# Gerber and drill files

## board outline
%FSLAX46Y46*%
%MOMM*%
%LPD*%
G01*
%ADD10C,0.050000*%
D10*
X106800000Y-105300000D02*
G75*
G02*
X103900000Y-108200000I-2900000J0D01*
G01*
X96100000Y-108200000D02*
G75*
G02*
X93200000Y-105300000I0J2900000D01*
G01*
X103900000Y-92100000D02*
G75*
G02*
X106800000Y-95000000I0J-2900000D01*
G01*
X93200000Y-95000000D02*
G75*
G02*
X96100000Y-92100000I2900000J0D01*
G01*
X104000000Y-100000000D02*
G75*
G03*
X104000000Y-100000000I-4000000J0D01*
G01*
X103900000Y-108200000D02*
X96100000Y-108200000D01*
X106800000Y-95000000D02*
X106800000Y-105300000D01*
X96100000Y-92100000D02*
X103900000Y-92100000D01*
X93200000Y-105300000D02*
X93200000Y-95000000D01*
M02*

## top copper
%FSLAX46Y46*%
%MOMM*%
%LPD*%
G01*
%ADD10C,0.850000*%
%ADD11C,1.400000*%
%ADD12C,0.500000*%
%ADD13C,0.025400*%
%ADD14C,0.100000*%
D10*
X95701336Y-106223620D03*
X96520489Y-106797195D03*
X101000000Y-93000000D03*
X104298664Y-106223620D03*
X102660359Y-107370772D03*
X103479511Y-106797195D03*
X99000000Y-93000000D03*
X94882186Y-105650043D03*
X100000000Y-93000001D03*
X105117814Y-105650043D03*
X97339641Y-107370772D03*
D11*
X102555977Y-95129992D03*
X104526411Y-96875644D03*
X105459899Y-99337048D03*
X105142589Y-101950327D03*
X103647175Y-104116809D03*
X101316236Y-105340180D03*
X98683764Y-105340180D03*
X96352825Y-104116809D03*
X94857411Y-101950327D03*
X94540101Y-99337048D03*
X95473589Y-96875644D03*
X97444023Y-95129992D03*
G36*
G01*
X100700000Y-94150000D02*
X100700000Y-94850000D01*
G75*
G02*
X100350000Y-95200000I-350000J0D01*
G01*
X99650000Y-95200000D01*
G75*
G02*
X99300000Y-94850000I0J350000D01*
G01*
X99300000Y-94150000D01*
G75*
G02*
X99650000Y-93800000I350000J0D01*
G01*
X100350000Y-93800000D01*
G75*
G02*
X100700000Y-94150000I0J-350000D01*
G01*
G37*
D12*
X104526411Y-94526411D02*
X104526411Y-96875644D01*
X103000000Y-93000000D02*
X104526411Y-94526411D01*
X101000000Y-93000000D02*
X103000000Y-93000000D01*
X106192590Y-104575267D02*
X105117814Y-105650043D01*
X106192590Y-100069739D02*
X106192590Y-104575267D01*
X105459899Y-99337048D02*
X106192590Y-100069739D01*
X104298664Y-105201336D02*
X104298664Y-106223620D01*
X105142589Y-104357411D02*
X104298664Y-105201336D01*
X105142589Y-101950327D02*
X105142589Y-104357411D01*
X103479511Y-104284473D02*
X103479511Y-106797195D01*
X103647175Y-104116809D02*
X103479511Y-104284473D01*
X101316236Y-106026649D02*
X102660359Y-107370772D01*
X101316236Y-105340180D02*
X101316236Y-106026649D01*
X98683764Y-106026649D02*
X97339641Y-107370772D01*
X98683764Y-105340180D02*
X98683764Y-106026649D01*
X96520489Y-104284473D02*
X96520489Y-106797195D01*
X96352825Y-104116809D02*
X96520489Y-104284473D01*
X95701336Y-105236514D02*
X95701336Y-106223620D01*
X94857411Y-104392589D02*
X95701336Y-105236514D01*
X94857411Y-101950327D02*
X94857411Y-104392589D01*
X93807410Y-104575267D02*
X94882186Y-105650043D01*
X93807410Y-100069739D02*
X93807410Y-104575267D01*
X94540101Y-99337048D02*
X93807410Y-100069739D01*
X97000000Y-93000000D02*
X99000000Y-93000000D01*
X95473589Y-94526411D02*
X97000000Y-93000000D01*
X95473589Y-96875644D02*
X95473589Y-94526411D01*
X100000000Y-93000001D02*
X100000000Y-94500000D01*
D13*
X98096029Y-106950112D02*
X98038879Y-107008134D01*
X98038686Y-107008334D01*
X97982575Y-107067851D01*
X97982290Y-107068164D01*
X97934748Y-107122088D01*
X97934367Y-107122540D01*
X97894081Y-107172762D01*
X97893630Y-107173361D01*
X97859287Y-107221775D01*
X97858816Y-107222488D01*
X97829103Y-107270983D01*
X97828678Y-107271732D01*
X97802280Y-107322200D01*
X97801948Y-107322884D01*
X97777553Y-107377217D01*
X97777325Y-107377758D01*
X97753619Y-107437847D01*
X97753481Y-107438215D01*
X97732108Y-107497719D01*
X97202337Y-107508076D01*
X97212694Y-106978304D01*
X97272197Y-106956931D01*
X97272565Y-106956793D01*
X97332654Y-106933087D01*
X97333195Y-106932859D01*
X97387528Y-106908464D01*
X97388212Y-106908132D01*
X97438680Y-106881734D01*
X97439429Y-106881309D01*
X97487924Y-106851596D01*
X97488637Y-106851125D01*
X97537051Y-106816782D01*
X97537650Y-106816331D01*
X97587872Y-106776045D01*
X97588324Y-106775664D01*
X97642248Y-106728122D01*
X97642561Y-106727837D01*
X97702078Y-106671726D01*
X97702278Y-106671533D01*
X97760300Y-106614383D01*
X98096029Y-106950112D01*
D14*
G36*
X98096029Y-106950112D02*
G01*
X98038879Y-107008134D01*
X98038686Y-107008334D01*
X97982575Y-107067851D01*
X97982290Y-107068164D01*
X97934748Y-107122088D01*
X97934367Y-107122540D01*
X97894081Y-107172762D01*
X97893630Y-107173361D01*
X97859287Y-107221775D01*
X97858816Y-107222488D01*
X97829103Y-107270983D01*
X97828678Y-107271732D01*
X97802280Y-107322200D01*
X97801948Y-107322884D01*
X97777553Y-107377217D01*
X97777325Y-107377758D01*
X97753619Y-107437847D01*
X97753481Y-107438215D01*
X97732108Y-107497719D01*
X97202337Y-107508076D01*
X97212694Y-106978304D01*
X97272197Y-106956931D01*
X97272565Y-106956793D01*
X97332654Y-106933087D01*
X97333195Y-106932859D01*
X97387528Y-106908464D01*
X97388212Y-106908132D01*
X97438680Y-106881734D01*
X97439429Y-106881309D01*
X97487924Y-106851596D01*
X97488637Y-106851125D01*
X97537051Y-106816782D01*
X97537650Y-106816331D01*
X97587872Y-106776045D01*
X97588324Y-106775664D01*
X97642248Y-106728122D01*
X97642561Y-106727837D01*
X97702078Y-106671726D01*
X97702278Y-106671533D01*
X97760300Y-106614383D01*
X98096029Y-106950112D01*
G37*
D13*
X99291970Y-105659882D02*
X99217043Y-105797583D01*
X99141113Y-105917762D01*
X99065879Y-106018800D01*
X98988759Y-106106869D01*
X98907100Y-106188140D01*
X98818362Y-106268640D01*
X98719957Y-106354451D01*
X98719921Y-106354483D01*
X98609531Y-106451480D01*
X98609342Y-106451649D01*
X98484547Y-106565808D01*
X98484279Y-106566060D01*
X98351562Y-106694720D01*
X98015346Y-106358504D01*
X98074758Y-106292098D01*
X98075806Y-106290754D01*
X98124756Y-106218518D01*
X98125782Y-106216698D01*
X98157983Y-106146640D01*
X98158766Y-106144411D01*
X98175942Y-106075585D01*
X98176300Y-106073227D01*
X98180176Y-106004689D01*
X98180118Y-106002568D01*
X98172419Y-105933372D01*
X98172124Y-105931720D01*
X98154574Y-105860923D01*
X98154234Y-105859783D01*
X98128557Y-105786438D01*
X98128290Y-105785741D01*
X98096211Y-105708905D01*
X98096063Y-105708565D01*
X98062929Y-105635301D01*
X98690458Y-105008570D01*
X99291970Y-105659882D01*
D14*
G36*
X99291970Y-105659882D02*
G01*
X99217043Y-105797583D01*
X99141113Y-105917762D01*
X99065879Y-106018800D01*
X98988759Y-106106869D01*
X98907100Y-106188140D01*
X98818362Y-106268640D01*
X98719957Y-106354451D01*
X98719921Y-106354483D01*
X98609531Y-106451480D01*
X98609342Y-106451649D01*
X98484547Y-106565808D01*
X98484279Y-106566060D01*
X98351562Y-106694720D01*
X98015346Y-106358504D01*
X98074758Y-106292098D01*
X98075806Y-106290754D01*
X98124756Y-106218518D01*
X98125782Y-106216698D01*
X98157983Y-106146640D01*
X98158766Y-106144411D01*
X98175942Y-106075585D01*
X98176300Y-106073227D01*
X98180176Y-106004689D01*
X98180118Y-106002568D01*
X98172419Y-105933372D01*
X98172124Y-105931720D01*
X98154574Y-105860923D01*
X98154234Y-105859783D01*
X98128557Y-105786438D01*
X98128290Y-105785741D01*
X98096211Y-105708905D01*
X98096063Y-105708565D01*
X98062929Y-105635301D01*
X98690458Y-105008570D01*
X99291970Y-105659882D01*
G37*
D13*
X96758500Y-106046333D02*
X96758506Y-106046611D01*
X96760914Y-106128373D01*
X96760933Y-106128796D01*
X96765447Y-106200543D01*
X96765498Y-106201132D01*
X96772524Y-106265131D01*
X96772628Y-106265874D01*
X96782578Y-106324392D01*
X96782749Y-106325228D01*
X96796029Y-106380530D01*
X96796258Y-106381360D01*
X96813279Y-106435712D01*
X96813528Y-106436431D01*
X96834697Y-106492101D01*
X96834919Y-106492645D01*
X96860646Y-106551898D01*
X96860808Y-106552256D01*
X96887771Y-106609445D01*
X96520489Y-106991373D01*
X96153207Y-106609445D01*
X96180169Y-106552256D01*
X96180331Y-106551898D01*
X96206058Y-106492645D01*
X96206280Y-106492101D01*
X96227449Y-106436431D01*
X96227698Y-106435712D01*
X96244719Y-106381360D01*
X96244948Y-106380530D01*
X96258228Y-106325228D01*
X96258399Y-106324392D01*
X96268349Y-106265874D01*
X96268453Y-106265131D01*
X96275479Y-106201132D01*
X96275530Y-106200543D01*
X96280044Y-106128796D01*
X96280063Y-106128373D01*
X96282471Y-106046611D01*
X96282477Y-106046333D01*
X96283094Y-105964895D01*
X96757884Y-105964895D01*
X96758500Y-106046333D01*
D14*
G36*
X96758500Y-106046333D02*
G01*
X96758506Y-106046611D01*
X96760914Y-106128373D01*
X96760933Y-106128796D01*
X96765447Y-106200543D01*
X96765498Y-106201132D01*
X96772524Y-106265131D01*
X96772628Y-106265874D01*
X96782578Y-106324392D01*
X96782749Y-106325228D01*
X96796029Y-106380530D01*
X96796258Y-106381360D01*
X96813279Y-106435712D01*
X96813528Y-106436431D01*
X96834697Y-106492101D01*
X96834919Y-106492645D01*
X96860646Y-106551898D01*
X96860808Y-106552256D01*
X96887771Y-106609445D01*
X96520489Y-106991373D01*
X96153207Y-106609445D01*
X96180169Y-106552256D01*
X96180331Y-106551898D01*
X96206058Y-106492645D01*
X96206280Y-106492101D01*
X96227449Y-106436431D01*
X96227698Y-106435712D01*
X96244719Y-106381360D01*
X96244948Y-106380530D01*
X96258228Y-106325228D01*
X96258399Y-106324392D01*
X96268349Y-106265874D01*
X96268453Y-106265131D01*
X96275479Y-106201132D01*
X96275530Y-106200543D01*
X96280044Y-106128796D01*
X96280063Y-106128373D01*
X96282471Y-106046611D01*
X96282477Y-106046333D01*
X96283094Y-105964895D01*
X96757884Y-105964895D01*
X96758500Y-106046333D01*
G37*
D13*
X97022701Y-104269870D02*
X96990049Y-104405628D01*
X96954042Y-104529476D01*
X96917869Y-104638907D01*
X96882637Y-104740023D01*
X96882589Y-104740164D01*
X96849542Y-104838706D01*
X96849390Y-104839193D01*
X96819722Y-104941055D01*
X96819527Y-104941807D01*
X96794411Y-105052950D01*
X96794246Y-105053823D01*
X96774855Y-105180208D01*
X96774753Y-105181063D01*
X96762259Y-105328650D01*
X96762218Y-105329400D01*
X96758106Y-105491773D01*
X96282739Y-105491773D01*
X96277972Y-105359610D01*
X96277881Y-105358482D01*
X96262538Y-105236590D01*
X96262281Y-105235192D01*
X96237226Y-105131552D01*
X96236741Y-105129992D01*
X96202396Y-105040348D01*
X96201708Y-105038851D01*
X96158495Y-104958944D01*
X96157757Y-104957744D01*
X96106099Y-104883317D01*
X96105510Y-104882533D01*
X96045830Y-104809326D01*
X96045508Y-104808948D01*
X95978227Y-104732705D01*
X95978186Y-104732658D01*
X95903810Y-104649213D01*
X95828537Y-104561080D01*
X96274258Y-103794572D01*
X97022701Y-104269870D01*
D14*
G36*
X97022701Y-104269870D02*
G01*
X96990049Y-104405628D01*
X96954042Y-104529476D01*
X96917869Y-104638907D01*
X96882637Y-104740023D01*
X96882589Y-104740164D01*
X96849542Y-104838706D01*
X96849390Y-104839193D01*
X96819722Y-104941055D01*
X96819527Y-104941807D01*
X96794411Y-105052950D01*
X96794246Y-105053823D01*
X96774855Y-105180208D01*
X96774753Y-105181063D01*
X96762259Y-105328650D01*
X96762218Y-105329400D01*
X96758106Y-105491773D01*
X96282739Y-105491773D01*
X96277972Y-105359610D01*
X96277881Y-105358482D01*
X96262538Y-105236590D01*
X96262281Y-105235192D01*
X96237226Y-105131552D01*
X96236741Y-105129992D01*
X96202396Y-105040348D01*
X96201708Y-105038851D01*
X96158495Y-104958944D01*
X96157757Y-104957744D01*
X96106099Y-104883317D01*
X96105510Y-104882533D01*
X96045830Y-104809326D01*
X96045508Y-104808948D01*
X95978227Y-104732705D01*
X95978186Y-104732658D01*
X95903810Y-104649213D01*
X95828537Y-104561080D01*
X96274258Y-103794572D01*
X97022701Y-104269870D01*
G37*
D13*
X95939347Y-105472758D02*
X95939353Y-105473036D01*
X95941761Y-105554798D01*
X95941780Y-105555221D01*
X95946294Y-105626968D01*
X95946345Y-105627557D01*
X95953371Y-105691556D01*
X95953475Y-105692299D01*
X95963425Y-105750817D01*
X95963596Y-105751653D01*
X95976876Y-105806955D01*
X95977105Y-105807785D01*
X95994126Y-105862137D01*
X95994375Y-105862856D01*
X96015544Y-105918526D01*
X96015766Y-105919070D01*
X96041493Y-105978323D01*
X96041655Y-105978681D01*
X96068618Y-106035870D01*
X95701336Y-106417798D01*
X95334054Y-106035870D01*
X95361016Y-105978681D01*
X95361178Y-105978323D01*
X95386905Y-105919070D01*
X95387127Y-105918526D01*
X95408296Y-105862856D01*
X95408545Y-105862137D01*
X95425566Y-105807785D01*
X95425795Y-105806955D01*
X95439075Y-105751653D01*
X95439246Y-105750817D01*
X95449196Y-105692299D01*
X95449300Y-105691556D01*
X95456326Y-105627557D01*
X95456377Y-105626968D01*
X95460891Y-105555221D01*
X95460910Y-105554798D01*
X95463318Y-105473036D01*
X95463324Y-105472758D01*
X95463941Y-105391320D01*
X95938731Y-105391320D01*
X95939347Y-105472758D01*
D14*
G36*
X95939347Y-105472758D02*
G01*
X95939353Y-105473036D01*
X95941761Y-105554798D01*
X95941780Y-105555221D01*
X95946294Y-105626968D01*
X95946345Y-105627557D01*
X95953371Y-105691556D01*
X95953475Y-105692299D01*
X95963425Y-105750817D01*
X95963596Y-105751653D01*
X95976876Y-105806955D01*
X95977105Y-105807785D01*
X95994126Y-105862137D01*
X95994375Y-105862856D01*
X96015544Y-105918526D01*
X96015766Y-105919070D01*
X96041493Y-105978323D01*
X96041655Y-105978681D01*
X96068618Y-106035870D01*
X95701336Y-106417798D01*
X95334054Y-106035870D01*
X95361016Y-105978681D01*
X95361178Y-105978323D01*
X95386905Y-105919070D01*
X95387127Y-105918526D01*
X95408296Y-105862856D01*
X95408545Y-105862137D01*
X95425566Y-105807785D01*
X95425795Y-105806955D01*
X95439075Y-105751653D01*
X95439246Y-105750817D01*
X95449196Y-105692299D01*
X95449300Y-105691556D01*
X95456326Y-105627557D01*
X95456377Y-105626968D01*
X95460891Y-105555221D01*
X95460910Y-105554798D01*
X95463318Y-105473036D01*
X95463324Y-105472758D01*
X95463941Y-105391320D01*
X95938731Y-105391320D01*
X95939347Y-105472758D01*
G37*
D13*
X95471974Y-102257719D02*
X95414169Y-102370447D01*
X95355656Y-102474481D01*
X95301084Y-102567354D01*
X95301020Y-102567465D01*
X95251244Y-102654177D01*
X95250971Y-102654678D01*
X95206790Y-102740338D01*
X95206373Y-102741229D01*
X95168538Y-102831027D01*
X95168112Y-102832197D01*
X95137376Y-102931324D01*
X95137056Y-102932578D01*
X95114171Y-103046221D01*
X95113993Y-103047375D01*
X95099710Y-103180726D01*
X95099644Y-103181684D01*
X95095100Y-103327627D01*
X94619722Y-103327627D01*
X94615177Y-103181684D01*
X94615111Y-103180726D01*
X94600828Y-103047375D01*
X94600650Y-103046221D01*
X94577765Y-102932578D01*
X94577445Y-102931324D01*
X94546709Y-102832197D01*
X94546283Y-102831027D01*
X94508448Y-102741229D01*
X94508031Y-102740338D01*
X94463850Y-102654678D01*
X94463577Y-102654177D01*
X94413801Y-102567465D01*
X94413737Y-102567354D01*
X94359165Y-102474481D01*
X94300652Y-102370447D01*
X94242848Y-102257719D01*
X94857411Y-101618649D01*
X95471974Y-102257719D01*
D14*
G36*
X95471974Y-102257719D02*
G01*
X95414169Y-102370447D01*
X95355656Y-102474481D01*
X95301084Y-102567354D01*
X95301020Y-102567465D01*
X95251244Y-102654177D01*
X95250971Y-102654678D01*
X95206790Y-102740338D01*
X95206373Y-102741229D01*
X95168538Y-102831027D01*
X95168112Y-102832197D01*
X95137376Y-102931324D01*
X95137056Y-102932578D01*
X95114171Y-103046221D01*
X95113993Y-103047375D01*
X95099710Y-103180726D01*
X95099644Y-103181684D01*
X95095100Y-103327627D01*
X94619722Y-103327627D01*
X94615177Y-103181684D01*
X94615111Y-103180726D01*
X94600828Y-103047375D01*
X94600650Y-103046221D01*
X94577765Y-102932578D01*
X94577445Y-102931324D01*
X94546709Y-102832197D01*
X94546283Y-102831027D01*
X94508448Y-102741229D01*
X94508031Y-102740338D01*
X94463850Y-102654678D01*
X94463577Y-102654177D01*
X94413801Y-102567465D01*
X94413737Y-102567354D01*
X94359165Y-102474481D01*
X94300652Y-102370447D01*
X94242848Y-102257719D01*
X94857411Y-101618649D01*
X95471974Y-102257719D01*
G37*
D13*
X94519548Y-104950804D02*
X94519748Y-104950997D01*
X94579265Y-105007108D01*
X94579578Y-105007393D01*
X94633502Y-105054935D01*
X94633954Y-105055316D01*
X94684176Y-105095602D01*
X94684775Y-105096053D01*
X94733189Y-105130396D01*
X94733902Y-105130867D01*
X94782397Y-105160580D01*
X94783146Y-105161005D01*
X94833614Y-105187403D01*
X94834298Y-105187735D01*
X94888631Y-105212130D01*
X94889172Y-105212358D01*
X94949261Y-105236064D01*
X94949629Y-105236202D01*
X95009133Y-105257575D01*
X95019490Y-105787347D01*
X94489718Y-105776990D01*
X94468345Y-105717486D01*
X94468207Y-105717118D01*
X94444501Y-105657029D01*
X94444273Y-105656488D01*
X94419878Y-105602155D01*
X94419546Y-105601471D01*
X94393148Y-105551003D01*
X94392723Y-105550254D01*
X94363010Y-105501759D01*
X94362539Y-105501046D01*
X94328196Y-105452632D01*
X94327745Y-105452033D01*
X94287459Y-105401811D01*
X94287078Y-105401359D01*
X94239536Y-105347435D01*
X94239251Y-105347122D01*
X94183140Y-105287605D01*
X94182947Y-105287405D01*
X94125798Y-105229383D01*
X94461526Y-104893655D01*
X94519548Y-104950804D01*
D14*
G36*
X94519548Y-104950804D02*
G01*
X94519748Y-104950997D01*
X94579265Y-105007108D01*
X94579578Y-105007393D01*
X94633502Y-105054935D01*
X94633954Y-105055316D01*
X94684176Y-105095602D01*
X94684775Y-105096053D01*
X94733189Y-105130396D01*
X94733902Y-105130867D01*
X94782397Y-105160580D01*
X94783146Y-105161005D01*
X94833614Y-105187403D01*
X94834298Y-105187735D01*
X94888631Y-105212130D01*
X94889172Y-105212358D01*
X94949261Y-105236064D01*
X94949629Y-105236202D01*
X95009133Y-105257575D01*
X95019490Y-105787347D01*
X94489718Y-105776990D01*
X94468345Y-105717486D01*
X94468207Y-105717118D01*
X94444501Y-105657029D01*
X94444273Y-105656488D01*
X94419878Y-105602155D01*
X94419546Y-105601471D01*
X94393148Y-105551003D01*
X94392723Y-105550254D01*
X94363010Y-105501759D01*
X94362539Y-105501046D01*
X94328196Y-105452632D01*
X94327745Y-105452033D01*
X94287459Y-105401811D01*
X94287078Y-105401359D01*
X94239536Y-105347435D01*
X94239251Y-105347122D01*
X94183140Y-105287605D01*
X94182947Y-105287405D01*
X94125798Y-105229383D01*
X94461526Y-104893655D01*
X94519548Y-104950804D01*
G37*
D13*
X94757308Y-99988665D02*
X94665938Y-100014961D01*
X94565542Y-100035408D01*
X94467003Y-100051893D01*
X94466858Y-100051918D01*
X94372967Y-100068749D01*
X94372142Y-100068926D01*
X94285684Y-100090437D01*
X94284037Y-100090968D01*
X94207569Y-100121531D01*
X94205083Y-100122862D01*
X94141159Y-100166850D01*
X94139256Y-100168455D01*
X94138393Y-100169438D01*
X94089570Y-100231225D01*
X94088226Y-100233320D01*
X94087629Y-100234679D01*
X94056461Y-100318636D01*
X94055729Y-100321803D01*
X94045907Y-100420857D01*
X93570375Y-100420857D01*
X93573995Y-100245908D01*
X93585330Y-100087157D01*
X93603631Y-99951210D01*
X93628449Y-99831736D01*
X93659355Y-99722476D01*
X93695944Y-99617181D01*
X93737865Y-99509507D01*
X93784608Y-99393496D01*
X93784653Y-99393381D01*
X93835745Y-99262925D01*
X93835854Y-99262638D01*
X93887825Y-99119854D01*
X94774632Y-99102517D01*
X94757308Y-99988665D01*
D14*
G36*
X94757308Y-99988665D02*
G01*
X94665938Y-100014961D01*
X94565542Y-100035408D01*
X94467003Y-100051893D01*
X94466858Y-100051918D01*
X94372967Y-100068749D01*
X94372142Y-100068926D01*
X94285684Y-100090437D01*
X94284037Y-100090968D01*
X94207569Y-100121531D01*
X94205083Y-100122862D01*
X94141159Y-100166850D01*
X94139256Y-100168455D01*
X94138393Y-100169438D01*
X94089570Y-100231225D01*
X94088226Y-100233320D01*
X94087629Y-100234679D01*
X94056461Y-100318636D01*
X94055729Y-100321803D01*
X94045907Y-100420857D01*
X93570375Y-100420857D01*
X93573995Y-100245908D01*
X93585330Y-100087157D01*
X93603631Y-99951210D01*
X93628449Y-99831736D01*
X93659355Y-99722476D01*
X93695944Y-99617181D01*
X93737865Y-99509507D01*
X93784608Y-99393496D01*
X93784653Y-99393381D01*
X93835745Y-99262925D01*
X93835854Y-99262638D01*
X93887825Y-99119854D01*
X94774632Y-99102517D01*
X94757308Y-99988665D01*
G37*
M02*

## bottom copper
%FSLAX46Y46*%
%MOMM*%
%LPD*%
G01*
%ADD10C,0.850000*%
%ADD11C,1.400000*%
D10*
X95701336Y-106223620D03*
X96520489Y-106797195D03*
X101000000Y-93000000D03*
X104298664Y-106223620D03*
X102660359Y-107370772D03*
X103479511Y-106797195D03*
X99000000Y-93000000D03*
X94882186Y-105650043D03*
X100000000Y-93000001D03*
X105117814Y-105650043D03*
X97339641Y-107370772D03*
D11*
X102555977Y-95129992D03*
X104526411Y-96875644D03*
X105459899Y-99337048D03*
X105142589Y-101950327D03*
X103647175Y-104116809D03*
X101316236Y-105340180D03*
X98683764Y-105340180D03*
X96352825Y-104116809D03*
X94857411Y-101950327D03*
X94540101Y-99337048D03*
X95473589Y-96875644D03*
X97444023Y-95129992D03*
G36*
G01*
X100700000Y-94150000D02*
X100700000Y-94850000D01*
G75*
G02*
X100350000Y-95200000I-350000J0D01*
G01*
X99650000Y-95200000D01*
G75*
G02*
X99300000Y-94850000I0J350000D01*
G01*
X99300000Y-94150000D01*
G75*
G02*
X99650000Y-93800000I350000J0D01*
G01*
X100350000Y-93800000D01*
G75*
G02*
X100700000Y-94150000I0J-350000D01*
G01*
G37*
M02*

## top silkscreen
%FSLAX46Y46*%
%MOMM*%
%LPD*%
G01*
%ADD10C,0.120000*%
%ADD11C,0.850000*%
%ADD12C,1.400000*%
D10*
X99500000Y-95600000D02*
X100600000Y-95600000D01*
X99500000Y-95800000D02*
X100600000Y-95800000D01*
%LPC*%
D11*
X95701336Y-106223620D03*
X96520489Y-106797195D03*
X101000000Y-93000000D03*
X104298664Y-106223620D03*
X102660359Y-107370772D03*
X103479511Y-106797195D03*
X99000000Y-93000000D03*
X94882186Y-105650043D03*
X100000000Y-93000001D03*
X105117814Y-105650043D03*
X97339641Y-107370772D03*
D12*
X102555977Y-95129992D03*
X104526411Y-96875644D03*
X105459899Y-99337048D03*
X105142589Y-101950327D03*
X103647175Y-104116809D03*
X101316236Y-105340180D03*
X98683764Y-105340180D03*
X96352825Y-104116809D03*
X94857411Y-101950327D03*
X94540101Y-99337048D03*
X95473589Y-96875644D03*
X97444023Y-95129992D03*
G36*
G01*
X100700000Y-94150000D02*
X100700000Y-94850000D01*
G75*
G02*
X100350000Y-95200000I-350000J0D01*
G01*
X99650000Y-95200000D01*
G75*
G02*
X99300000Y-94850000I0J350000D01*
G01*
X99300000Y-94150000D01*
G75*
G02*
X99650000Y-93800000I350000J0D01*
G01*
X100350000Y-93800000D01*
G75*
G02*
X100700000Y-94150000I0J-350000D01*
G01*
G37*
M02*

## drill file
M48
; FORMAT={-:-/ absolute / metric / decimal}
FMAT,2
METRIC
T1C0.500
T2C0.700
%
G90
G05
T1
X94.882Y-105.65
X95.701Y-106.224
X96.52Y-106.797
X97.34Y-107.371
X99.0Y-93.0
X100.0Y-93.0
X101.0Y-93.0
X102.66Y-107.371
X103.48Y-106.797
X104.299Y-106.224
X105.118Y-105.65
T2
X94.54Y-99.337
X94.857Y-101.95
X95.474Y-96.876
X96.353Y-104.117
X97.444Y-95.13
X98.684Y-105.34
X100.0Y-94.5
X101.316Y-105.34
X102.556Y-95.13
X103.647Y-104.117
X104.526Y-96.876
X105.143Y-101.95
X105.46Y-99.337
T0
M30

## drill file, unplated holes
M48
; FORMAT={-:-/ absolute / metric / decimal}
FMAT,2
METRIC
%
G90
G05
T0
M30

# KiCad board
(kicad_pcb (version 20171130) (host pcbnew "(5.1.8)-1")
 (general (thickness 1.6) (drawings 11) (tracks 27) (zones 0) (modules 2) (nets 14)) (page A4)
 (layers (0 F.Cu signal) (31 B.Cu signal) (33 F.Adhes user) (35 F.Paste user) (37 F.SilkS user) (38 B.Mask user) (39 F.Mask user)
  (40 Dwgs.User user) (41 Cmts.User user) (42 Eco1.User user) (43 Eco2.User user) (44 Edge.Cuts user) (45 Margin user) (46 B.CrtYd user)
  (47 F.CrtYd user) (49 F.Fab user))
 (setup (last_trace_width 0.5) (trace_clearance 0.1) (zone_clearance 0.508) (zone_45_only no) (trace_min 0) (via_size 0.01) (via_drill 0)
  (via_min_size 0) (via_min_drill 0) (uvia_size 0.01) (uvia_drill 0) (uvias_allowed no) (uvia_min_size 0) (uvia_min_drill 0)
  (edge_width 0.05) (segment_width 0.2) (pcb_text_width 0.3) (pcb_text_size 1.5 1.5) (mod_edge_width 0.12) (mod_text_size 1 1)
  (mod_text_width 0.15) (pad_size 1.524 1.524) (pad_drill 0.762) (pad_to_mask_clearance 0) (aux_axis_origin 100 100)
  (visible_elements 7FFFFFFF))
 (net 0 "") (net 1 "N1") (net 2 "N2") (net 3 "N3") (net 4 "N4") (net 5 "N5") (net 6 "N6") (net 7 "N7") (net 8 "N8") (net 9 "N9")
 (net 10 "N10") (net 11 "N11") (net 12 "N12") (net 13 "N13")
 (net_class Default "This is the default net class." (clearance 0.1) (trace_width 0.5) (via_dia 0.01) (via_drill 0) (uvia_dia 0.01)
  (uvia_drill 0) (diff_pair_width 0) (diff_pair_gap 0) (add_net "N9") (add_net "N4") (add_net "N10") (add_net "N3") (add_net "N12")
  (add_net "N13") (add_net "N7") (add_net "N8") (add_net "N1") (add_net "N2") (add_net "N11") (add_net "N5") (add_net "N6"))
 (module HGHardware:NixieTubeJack (layer F.Cu) (at 100 100)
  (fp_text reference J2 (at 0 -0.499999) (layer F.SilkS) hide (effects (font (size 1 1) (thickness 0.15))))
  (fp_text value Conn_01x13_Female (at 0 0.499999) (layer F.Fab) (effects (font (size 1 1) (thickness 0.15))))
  (pad 5 thru_hole circle (at -4.298664 6.22362 325) (size 0.85 0.85) (drill 0.5) (layers *.Cu *.Mask) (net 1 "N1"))
  (pad 6 thru_hole circle (at -3.479511 6.797195 235) (size 0.85 0.85) (drill 0.5) (layers *.Cu *.Mask) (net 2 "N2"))
  (pad 12 thru_hole circle (at 1 -7 270) (size 0.85 0.85) (drill 0.5) (layers *.Cu *.Mask) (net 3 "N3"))
  (pad 10 thru_hole circle (at 4.298664 6.22362 230) (size 0.85 0.85) (drill 0.5) (layers *.Cu *.Mask) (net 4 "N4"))
  (pad 8 thru_hole circle (at 2.660359 7.370772 140) (size 0.85 0.85) (drill 0.5) (layers *.Cu *.Mask) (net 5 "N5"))
  (pad 9 thru_hole circle (at 3.479511 6.797195 140) (size 0.85 0.85) (drill 0.5) (layers *.Cu *.Mask) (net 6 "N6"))
  (pad 3 thru_hole circle (at -1 -7 270) (size 0.85 0.85) (drill 0.5) (layers *.Cu *.Mask) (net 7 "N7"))
  (pad 4 thru_hole circle (at -5.117814 5.650043 325) (size 0.85 0.85) (drill 0.5) (layers *.Cu *.Mask) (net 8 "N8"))
  (pad 1 thru_hole circle (at 0 -6.999999 180) (size 0.85 0.85) (drill 0.5) (layers *.Cu *.Mask) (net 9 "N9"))
  (pad 11 thru_hole circle (at 5.117814 5.650043 230) (size 0.85 0.85) (drill 0.5) (layers *.Cu *.Mask) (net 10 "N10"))
  (pad 7 thru_hole circle (at -2.660359 7.370772 235) (size 0.85 0.85) (drill 0.5) (layers *.Cu *.Mask) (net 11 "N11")))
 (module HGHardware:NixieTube (layer F.Cu) (at 100 100 180)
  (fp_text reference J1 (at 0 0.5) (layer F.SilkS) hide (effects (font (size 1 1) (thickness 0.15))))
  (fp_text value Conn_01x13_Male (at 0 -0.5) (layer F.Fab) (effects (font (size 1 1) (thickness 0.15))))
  (pad 13 thru_hole circle (at -2.555977 4.870008 180) (size 1.4 1.4) (drill 0.7) (layers *.Cu *.Mask) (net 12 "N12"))
  (pad 12 thru_hole circle (at -4.526411 3.124356 180) (size 1.4 1.4) (drill 0.7) (layers *.Cu *.Mask) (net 3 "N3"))
  (pad 11 thru_hole circle (at -5.459899 0.662952 180) (size 1.4 1.4) (drill 0.7) (layers *.Cu *.Mask) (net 10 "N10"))
  (pad 10 thru_hole circle (at -5.142589 -1.950327 180) (size 1.4 1.4) (drill 0.7) (layers *.Cu *.Mask) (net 4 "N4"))
  (pad 9 thru_hole circle (at -3.647175 -4.116809 180) (size 1.4 1.4) (drill 0.7) (layers *.Cu *.Mask) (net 6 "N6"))
  (pad 8 thru_hole circle (at -1.316236 -5.34018 180) (size 1.4 1.4) (drill 0.7) (layers *.Cu *.Mask) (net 5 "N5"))
  (pad 7 thru_hole circle (at 1.316236 -5.34018 180) (size 1.4 1.4) (drill 0.7) (layers *.Cu *.Mask) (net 11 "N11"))
  (pad 6 thru_hole circle (at 3.647175 -4.116809 180) (size 1.4 1.4) (drill 0.7) (layers *.Cu *.Mask) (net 2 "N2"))
  (pad 5 thru_hole circle (at 5.142589 -1.950327 180) (size 1.4 1.4) (drill 0.7) (layers *.Cu *.Mask) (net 1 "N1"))
  (pad 4 thru_hole circle (at 5.459899 0.662952 180) (size 1.4 1.4) (drill 0.7) (layers *.Cu *.Mask) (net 8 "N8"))
  (pad 3 thru_hole circle (at 4.526411 3.124356 180) (size 1.4 1.4) (drill 0.7) (layers *.Cu *.Mask) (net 7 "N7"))
  (pad 2 thru_hole circle (at 2.555977 4.870008 180) (size 1.4 1.4) (drill 0.7) (layers *.Cu *.Mask) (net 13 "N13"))
  (pad 1 thru_hole roundrect (at 0 5.5 180) (size 1.4 1.4) (drill 0.7) (layers *.Cu *.Mask) (roundrect_rratio 0.25) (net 9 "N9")))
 (gr_arc (start 103.9 105.3) (end 103.9 108.2) (angle -90) (layer Edge.Cuts) (width 0.05))
 (gr_arc (start 96.1 105.3) (end 93.2 105.3) (angle -90) (layer Edge.Cuts) (width 0.05))
 (gr_arc (start 103.9 95) (end 106.8 95) (angle -90) (layer Edge.Cuts) (width 0.05))
 (gr_arc (start 96.1 95) (end 96.1 92.1) (angle -90) (layer Edge.Cuts) (width 0.05))
 (gr_circle (center 100 100) (end 104 100) (layer Edge.Cuts) (width 0.05))
 (gr_line (start 103.9 108.2) (end 96.1 108.2) (layer Edge.Cuts) (width 0.05))
 (gr_line (start 106.8 95) (end 106.8 105.3) (layer Edge.Cuts) (width 0.05))
 (gr_line (start 96.1 92.1) (end 103.9 92.1) (layer Edge.Cuts) (width 0.05))
 (gr_line (start 93.2 105.3) (end 93.2 95) (layer Edge.Cuts) (width 0.05))
 (gr_line (start 99.5 95.6) (end 100.6 95.6) (layer F.SilkS) (width 0.12))
 (gr_line (start 99.5 95.8) (end 100.6 95.8) (layer F.SilkS) (width 0.12))
 (segment (start 104.526411 94.526411) (end 104.526411 96.875644) (width 0.5) (layer F.Cu) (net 3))
 (segment (start 103 93) (end 104.526411 94.526411) (width 0.5) (layer F.Cu) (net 3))
 (segment (start 101 93) (end 103 93) (width 0.5) (layer F.Cu) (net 3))
 (segment (start 106.19259 104.575267) (end 105.117814 105.650043) (width 0.5) (layer F.Cu) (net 10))
 (segment (start 106.19259 100.069739) (end 106.19259 104.575267) (width 0.5) (layer F.Cu) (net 10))
 (segment (start 105.459899 99.337048) (end 106.19259 100.069739) (width 0.5) (layer F.Cu) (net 10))
 (segment (start 104.298664 105.201336) (end 104.298664 106.22362) (width 0.5) (layer F.Cu) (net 4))
 (segment (start 105.142589 104.357411) (end 104.298664 105.201336) (width 0.5) (layer F.Cu) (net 4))
 (segment (start 105.142589 101.950327) (end 105.142589 104.357411) (width 0.5) (layer F.Cu) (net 4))
 (segment (start 103.479511 104.284473) (end 103.479511 106.797195) (width 0.5) (layer F.Cu) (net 6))
 (segment (start 103.647175 104.116809) (end 103.479511 104.284473) (width 0.5) (layer F.Cu) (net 6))
 (segment (start 101.316236 106.026649) (end 102.660359 107.370772) (width 0.5) (layer F.Cu) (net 5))
 (segment (start 101.316236 105.34018) (end 101.316236 106.026649) (width 0.5) (layer F.Cu) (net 5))
 (segment (start 98.683764 106.026649) (end 97.339641 107.370772) (width 0.5) (layer F.Cu) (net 11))
 (segment (start 98.683764 105.34018) (end 98.683764 106.026649) (width 0.5) (layer F.Cu) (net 11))
 (segment (start 96.520489 104.284473) (end 96.520489 106.797195) (width 0.5) (layer F.Cu) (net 2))
 (segment (start 96.352825 104.116809) (end 96.520489 104.284473) (width 0.5) (layer F.Cu) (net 2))
 (segment (start 95.701336 105.236514) (end 95.701336 106.22362) (width 0.5) (layer F.Cu) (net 1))
 (segment (start 94.857411 104.392589) (end 95.701336 105.236514) (width 0.5) (layer F.Cu) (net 1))
 (segment (start 94.857411 101.950327) (end 94.857411 104.392589) (width 0.5) (layer F.Cu) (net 1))
 (segment (start 93.80741 104.575267) (end 94.882186 105.650043) (width 0.5) (layer F.Cu) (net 8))
 (segment (start 93.80741 100.069739) (end 93.80741 104.575267) (width 0.5) (layer F.Cu) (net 8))
 (segment (start 94.540101 99.337048) (end 93.80741 100.069739) (width 0.5) (layer F.Cu) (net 8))
 (segment (start 97 93) (end 99 93) (width 0.5) (layer F.Cu) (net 7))
 (segment (start 95.473589 94.526411) (end 97 93) (width 0.5) (layer F.Cu) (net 7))
 (segment (start 95.473589 96.875644) (end 95.473589 94.526411) (width 0.5) (layer F.Cu) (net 7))
 (segment (start 100 93.000001) (end 100 94.5) (width 0.5) (layer F.Cu) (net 9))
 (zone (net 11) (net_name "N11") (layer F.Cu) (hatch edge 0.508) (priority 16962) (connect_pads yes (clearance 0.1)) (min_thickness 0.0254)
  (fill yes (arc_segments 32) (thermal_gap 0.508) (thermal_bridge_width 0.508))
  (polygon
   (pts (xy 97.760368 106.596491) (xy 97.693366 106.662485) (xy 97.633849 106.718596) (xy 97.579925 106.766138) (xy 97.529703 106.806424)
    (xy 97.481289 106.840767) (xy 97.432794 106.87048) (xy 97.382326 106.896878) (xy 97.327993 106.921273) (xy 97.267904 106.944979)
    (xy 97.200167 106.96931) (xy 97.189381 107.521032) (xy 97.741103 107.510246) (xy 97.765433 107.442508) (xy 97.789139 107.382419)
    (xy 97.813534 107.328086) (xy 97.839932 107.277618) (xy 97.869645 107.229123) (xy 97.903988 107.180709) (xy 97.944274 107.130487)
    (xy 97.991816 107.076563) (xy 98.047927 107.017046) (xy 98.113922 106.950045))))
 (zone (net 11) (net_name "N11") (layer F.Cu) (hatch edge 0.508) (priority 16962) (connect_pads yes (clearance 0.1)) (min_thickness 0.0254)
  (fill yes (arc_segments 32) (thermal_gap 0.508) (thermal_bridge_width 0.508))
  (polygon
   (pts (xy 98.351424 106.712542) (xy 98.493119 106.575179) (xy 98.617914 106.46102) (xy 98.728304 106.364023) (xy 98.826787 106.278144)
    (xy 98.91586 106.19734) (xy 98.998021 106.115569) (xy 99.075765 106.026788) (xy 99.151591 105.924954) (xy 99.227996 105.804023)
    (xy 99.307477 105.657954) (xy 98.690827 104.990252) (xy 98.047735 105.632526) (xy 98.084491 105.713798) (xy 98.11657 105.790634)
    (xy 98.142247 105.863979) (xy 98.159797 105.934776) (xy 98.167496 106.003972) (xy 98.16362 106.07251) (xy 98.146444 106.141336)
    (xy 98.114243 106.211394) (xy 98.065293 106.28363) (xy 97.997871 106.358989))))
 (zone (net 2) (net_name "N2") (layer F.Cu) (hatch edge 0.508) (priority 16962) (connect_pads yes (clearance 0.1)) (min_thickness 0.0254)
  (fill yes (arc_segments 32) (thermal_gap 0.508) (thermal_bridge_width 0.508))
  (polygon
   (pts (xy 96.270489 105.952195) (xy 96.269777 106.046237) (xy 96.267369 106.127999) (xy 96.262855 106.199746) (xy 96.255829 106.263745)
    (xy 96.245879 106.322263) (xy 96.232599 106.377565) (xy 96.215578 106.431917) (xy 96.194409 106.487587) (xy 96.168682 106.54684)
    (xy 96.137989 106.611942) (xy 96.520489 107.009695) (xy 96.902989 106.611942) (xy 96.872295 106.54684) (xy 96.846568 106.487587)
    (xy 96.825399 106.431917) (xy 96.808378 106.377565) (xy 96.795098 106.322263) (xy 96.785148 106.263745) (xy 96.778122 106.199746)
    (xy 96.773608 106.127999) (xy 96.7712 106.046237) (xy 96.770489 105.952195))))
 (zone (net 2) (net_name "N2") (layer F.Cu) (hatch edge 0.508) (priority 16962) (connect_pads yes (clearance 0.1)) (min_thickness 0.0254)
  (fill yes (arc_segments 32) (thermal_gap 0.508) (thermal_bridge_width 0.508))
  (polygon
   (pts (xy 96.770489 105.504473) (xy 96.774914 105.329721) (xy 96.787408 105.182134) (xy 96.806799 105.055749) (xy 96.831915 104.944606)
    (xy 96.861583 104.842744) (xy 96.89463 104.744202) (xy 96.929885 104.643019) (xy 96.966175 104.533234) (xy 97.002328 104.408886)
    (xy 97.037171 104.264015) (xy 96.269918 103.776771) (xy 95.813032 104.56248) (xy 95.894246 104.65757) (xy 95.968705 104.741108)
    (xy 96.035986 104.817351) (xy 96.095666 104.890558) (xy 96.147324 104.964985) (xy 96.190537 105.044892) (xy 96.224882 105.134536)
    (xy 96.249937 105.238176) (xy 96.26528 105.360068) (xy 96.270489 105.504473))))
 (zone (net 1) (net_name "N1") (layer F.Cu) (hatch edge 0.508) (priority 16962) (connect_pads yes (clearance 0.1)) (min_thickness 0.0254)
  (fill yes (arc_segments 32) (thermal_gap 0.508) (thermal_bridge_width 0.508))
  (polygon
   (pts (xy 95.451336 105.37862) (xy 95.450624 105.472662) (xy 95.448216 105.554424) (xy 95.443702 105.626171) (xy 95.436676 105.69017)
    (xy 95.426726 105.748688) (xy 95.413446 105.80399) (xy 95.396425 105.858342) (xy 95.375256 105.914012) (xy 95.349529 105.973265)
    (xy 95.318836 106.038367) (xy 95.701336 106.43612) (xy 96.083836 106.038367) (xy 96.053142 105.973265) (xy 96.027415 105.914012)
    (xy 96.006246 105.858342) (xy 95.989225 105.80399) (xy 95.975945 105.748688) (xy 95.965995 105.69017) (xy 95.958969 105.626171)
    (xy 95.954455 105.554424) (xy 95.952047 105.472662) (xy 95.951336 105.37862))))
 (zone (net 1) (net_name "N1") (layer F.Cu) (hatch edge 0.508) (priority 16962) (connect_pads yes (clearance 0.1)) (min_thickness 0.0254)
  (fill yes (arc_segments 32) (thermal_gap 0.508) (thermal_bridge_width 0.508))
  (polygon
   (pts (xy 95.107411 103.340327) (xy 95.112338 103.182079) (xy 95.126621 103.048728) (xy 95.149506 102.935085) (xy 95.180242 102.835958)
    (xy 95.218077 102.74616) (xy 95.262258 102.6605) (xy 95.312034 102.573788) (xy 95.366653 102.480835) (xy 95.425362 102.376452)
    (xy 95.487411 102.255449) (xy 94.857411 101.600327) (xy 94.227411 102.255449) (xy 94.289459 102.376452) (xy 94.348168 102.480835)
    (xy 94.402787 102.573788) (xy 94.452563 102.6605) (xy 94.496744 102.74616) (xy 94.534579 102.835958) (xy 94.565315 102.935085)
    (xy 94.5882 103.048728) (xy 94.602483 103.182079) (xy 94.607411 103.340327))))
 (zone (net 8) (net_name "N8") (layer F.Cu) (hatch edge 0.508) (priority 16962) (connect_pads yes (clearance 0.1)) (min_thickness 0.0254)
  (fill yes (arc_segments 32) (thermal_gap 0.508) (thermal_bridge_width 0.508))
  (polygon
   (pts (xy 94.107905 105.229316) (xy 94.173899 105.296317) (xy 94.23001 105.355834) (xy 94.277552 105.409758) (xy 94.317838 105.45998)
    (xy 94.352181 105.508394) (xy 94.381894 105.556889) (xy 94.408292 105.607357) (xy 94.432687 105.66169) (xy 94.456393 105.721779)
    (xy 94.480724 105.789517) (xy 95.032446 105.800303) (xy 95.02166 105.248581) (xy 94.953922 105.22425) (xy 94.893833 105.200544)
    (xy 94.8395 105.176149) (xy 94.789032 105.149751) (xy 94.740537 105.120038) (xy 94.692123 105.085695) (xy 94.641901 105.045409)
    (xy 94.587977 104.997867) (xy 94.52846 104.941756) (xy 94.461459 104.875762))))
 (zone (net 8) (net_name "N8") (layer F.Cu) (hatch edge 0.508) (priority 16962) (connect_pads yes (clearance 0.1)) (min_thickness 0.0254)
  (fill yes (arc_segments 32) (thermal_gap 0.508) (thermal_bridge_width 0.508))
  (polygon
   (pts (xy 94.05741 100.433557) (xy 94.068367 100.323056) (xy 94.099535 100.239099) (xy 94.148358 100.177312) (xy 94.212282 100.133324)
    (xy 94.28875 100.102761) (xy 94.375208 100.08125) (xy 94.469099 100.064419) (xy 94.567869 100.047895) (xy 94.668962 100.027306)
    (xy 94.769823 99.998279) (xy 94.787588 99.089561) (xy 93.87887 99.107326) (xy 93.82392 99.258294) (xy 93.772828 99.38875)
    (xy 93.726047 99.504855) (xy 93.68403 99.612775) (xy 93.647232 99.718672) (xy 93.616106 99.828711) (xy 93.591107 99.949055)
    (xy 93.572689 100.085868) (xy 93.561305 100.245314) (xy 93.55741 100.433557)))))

